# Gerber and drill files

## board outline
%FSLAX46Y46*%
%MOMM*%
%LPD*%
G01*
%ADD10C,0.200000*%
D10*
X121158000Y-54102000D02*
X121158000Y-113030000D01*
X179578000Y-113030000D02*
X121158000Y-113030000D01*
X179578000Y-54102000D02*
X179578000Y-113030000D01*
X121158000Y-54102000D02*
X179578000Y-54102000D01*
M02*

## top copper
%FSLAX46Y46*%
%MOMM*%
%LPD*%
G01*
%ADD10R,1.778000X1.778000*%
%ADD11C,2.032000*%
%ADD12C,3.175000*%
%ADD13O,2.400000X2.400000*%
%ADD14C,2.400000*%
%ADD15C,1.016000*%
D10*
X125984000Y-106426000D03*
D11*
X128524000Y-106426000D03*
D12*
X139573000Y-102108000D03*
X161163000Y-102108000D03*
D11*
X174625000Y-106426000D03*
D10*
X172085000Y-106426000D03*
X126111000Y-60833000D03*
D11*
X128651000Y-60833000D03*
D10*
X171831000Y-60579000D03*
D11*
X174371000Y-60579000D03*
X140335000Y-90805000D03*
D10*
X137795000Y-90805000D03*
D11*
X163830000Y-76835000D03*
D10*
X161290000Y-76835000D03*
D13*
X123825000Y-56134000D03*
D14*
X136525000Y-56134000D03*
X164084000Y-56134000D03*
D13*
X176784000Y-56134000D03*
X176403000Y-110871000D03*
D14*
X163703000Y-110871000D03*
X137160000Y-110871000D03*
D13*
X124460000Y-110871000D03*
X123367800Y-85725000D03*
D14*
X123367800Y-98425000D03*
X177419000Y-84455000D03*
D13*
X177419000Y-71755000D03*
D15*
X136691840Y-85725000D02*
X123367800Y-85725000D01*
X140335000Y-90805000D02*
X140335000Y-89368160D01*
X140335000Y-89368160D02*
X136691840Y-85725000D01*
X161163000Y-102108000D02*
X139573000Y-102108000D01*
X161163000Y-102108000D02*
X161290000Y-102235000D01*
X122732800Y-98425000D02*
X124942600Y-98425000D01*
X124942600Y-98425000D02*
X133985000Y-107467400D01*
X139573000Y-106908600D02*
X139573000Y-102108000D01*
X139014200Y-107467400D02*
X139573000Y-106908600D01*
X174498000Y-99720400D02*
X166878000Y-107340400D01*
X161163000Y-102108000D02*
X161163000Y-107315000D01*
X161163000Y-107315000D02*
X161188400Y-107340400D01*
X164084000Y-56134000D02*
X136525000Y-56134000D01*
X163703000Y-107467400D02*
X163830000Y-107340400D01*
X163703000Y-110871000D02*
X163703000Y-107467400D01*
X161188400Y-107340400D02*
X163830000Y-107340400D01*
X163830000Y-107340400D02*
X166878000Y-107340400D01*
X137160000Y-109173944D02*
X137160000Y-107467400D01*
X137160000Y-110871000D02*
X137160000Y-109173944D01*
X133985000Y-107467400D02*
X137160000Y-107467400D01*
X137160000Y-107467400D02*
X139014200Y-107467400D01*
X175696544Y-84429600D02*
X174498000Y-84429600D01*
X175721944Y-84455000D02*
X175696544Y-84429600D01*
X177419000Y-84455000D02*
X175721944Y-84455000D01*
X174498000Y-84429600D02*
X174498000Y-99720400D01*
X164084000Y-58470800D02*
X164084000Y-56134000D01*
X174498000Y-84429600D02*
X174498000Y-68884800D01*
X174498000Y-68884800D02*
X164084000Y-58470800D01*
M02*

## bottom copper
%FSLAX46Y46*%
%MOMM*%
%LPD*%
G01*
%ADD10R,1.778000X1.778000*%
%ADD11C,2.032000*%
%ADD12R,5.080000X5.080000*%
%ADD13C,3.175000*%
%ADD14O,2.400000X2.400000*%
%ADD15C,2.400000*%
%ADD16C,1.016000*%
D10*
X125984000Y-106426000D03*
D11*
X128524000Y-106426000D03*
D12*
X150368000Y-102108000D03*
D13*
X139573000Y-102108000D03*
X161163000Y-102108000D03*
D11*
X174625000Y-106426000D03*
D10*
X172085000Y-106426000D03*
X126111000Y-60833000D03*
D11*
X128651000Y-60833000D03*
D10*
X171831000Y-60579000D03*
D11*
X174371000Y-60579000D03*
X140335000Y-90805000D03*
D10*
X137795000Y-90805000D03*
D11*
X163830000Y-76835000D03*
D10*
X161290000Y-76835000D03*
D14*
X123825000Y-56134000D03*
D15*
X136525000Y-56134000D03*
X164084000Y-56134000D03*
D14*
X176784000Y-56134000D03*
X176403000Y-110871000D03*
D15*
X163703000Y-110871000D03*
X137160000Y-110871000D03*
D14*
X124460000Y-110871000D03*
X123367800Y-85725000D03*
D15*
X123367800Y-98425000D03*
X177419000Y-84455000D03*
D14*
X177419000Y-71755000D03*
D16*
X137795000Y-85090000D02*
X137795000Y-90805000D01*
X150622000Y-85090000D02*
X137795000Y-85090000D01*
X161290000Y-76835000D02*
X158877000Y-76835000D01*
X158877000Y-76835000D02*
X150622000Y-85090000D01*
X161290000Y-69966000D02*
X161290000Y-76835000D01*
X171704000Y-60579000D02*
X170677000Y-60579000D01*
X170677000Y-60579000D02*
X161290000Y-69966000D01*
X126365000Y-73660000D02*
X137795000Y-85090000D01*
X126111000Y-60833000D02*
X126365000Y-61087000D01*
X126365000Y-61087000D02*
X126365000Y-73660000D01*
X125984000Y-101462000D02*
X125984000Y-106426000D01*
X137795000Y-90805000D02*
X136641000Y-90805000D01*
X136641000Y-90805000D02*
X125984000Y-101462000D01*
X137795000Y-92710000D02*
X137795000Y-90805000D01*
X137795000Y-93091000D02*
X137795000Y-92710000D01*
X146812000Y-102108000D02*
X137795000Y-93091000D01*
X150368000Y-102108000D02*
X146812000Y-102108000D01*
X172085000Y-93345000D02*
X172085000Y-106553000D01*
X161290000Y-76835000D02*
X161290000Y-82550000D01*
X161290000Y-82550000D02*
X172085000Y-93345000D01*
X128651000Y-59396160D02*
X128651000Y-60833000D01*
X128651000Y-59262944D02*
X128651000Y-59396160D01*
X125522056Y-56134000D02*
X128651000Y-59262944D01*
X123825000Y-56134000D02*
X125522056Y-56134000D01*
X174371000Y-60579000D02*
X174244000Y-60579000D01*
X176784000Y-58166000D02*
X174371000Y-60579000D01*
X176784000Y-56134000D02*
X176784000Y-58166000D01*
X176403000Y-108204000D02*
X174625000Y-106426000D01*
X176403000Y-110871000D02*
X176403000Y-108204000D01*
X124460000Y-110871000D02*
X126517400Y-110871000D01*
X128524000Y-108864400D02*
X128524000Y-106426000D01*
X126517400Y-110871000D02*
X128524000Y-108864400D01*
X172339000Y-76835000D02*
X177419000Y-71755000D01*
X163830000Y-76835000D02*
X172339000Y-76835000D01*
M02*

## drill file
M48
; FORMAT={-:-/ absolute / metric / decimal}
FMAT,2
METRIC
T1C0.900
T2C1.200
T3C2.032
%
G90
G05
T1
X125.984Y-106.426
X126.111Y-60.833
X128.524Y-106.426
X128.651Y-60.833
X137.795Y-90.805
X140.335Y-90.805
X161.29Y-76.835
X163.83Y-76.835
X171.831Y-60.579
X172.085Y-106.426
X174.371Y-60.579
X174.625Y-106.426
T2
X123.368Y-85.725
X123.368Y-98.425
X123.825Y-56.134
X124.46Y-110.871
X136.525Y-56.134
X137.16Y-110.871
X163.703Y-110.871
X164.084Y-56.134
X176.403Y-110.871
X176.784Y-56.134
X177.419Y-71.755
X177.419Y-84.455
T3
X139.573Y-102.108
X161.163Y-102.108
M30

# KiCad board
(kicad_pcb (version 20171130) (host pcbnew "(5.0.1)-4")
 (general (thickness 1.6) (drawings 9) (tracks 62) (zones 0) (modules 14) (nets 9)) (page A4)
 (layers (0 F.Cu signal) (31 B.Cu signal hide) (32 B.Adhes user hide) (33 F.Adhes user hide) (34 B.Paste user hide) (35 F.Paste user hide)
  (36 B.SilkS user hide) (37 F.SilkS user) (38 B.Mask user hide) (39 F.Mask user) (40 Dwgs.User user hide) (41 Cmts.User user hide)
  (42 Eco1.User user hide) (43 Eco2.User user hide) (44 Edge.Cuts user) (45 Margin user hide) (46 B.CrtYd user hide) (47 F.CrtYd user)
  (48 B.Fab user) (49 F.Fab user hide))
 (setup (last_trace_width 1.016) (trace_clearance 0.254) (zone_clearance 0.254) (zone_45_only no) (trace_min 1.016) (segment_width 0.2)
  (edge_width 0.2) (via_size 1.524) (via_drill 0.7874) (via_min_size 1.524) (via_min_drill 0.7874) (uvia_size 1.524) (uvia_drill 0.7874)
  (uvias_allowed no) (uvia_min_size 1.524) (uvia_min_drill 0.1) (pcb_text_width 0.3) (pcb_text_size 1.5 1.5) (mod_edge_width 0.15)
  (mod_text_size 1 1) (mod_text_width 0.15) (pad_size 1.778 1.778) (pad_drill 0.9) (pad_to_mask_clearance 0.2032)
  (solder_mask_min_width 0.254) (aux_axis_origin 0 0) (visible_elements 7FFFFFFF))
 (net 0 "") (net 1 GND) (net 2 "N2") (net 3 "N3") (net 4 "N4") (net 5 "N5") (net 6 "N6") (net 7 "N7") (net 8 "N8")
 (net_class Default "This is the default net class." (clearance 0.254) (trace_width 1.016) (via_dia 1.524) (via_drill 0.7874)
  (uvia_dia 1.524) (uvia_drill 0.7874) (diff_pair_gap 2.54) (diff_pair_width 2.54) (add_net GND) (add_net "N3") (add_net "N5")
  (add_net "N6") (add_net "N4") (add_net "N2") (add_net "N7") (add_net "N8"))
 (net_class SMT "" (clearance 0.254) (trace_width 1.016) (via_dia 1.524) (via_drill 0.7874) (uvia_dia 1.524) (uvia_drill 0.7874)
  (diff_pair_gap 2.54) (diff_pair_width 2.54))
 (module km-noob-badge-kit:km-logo (layer F.Cu) (at 150.368 83.566)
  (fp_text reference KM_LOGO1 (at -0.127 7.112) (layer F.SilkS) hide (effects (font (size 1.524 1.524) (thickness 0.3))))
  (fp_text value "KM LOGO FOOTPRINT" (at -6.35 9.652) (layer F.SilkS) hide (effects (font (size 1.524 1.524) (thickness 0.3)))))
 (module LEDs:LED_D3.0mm (layer F.Cu) (at 125.984 106.426)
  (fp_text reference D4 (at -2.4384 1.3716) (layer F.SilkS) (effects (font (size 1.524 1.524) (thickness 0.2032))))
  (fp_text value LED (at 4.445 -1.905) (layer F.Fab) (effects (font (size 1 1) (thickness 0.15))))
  (pad 1 thru_hole rect (at 0 0) (size 1.778 1.778) (drill 0.9) (layers *.Cu *.Mask) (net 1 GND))
  (pad 2 thru_hole circle (at 2.54 0) (size 2.032 2.032) (drill 0.9) (layers *.Cu *.Mask) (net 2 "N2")))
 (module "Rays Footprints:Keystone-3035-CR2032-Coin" (layer B.Cu) (at 150.368 102.108 180)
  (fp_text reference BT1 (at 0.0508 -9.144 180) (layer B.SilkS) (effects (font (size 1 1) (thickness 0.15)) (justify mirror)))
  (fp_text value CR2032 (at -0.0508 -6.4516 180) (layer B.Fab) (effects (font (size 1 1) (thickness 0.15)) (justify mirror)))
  (pad 2 smd rect (at 0 0 180) (size 5.08 5.08) (layers B.Cu B.Paste B.Mask) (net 1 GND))
  (pad 1 thru_hole circle (at 10.795 0 180) (size 3.175 3.175) (drill 2.032) (layers *.Cu *.Mask) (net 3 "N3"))
  (pad 1 thru_hole circle (at -10.795 0 90) (size 3.175 3.175) (drill 2.032) (layers *.Cu *.Mask) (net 3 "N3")))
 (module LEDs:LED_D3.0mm (layer F.Cu) (at 172.085 106.426)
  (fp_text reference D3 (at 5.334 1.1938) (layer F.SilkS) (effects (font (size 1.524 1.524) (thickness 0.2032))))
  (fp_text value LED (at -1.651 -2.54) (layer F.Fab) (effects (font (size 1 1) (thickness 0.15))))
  (pad 2 thru_hole circle (at 2.54 0) (size 2.032 2.032) (drill 0.9) (layers *.Cu *.Mask) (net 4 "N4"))
  (pad 1 thru_hole rect (at 0 0) (size 1.778 1.778) (drill 0.9) (layers *.Cu *.Mask) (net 1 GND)))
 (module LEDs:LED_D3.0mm (layer F.Cu) (at 126.111 60.833)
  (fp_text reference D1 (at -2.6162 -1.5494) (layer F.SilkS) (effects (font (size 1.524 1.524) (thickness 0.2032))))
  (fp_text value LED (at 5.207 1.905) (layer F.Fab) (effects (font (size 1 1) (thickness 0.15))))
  (pad 1 thru_hole rect (at 0 0) (size 1.778 1.778) (drill 0.9) (layers *.Cu *.Mask) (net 1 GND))
  (pad 2 thru_hole circle (at 2.54 0) (size 2.032 2.032) (drill 0.9) (layers *.Cu *.Mask) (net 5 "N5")))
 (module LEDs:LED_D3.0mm (layer F.Cu) (at 171.831 60.579)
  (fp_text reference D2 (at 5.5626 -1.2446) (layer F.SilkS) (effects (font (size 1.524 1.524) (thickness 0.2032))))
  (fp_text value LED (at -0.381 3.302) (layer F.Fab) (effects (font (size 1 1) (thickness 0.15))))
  (pad 1 thru_hole rect (at 0 0) (size 1.778 1.778) (drill 0.9) (layers *.Cu *.Mask) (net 1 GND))
  (pad 2 thru_hole circle (at 2.54 0) (size 2.032 2.032) (drill 0.9) (layers *.Cu *.Mask) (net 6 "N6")))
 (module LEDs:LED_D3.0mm (layer F.Cu) (at 137.795 90.805)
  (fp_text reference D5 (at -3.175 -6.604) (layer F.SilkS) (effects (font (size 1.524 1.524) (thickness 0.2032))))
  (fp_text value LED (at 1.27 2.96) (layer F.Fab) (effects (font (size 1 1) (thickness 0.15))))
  (pad 2 thru_hole circle (at 2.54 0) (size 2.032 2.032) (drill 0.9) (layers *.Cu *.Mask) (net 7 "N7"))
  (pad 1 thru_hole rect (at 0 0) (size 1.778 1.778) (drill 0.9) (layers *.Cu *.Mask) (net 1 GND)))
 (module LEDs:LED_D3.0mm (layer F.Cu) (at 161.29 76.835)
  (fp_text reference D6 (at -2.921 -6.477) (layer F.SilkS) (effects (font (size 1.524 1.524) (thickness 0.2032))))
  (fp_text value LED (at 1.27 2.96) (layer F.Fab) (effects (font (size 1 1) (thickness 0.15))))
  (pad 2 thru_hole circle (at 2.54 0) (size 2.032 2.032) (drill 0.9) (layers *.Cu *.Mask) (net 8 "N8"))
  (pad 1 thru_hole rect (at 0 0) (size 1.778 1.778) (drill 0.9) (layers *.Cu *.Mask) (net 1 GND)))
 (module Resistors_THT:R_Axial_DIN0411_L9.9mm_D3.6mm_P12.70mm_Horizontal (layer F.Cu) (at 136.525 56.134 180)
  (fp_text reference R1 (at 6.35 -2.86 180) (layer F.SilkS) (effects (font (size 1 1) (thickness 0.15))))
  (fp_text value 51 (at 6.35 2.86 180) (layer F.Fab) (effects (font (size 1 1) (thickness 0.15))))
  (pad 2 thru_hole oval (at 12.7 0 180) (size 2.4 2.4) (drill 1.2) (layers *.Cu *.Mask) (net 5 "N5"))
  (pad 1 thru_hole circle (at 0 0 180) (size 2.4 2.4) (drill 1.2) (layers *.Cu *.Mask) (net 3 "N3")))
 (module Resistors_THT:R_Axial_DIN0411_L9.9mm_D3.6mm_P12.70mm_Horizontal (layer F.Cu) (at 164.084 56.134)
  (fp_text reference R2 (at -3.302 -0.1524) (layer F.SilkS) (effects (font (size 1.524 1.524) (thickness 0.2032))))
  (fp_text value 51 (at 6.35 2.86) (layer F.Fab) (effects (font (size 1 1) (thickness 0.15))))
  (pad 1 thru_hole circle (at 0 0) (size 2.4 2.4) (drill 1.2) (layers *.Cu *.Mask) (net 3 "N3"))
  (pad 2 thru_hole oval (at 12.7 0) (size 2.4 2.4) (drill 1.2) (layers *.Cu *.Mask) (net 6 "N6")))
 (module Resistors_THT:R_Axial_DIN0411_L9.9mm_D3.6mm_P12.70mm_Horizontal (layer F.Cu) (at 163.703 110.871)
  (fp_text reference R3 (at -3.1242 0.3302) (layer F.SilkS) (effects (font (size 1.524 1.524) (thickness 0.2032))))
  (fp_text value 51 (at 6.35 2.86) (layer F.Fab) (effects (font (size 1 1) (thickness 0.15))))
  (pad 2 thru_hole oval (at 12.7 0) (size 2.4 2.4) (drill 1.2) (layers *.Cu *.Mask) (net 4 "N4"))
  (pad 1 thru_hole circle (at 0 0) (size 2.4 2.4) (drill 1.2) (layers *.Cu *.Mask) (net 3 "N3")))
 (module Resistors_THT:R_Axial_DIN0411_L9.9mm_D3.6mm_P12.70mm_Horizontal (layer F.Cu) (at 137.16 110.871 180)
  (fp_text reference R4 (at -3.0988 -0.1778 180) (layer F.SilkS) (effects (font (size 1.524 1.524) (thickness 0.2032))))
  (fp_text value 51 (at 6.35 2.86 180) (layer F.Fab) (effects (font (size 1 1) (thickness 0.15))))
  (pad 1 thru_hole circle (at 0 0 180) (size 2.4 2.4) (drill 1.2) (layers *.Cu *.Mask) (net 3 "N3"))
  (pad 2 thru_hole oval (at 12.7 0 180) (size 2.4 2.4) (drill 1.2) (layers *.Cu *.Mask) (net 2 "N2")))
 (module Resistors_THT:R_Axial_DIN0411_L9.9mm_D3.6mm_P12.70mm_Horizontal (layer F.Cu) (at 123.3678 98.425 90)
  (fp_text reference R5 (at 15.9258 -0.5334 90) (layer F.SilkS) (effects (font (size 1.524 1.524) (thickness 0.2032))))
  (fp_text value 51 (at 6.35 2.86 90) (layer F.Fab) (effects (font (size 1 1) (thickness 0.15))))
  (pad 2 thru_hole oval (at 12.7 0 90) (size 2.4 2.4) (drill 1.2) (layers *.Cu *.Mask) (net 7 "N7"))
  (pad 1 thru_hole circle (at 0 0 90) (size 2.4 2.4) (drill 1.2) (layers *.Cu *.Mask) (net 3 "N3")))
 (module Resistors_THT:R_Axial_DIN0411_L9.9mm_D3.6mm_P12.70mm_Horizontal (layer F.Cu) (at 177.419 84.455 90)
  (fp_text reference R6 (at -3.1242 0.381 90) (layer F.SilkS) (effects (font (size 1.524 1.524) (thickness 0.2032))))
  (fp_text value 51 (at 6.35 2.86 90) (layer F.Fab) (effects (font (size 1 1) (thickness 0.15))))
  (pad 1 thru_hole circle (at 0 0 90) (size 2.4 2.4) (drill 1.2) (layers *.Cu *.Mask) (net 3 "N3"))
  (pad 2 thru_hole oval (at 12.7 0 90) (size 2.4 2.4) (drill 1.2) (layers *.Cu *.Mask) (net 8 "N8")))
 (gr_line (start 121.158 54.102) (end 121.158 113.03) (layer Edge.Cuts) (width 0.2))
 (gr_line (start 179.578 113.03) (end 121.158 113.03) (layer Edge.Cuts) (width 0.2))
 (gr_line (start 179.578 54.102) (end 179.578 113.03) (layer Edge.Cuts) (width 0.2))
 (gr_line (start 121.158 54.102) (end 179.578 54.102) (layer Edge.Cuts) (width 0.2))
 (segment (start 137.795 85.09) (end 137.795 90.805) (width 1.016) (layer B.Cu) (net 1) (status 20))
 (segment (start 150.622 85.09) (end 137.795 85.09) (width 1.016) (layer B.Cu) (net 1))
 (segment (start 161.29 76.835) (end 158.877 76.835) (width 1.016) (layer B.Cu) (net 1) (status 10))
 (segment (start 158.877 76.835) (end 150.622 85.09) (width 1.016) (layer B.Cu) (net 1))
 (segment (start 161.29 69.966) (end 161.29 76.835) (width 1.016) (layer B.Cu) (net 1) (status 20))
 (segment (start 171.704 60.579) (end 170.677 60.579) (width 1.016) (layer B.Cu) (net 1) (status 10))
 (segment (start 170.677 60.579) (end 161.29 69.966) (width 1.016) (layer B.Cu) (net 1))
 (segment (start 126.365 73.66) (end 137.795 85.09) (width 1.016) (layer B.Cu) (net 1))
 (segment (start 126.111 60.833) (end 126.365 61.087) (width 1.016) (layer B.Cu) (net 1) (status 30))
 (segment (start 126.365 61.087) (end 126.365 73.66) (width 1.016) (layer B.Cu) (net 1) (status 10))
 (segment (start 125.984 101.462) (end 125.984 106.426) (width 1.016) (layer B.Cu) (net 1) (status 20))
 (segment (start 137.795 90.805) (end 136.641 90.805) (width 1.016) (layer B.Cu) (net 1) (status 10))
 (segment (start 136.641 90.805) (end 125.984 101.462) (width 1.016) (layer B.Cu) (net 1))
 (segment (start 137.795 92.71) (end 137.795 90.805) (width 1.016) (layer B.Cu) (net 1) (status 20))
 (segment (start 137.795 93.091) (end 137.795 92.71) (width 1.016) (layer B.Cu) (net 1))
 (segment (start 146.812 102.108) (end 137.795 93.091) (width 1.016) (layer B.Cu) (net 1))
 (segment (start 150.368 102.108) (end 146.812 102.108) (width 1.016) (layer B.Cu) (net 1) (status 10))
 (segment (start 172.085 93.345) (end 172.085 106.553) (width 1.016) (layer B.Cu) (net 1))
 (segment (start 161.29 76.835) (end 161.29 82.55) (width 1.016) (layer B.Cu) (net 1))
 (segment (start 161.29 82.55) (end 172.085 93.345) (width 1.016) (layer B.Cu) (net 1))
 (segment (start 128.651 59.39616) (end 128.651 60.833) (width 1.016) (layer B.Cu) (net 5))
 (segment (start 128.651 59.262944) (end 128.651 59.39616) (width 1.016) (layer B.Cu) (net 5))
 (segment (start 125.522056 56.134) (end 128.651 59.262944) (width 1.016) (layer B.Cu) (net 5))
 (segment (start 123.825 56.134) (end 125.522056 56.134) (width 1.016) (layer B.Cu) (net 5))
 (segment (start 174.371 60.579) (end 174.244 60.579) (width 1.016) (layer B.Cu) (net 6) (status 30))
 (segment (start 176.784 58.166) (end 174.371 60.579) (width 1.016) (layer B.Cu) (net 6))
 (segment (start 176.784 56.134) (end 176.784 58.166) (width 1.016) (layer B.Cu) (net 6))
 (segment (start 176.403 108.204) (end 174.625 106.426) (width 1.016) (layer B.Cu) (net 4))
 (segment (start 176.403 110.871) (end 176.403 108.204) (width 1.016) (layer B.Cu) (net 4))
 (segment (start 124.46 110.871) (end 126.5174 110.871) (width 1.016) (layer B.Cu) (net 2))
 (segment (start 128.524 108.8644) (end 128.524 106.426) (width 1.016) (layer B.Cu) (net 2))
 (segment (start 126.5174 110.871) (end 128.524 108.8644) (width 1.016) (layer B.Cu) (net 2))
 (segment (start 136.69184 85.725) (end 123.3678 85.725) (width 1.016) (layer F.Cu) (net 7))
 (segment (start 140.335 90.805) (end 140.335 89.36816) (width 1.016) (layer F.Cu) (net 7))
 (segment (start 140.335 89.36816) (end 136.69184 85.725) (width 1.016) (layer F.Cu) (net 7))
 (segment (start 172.339 76.835) (end 177.419 71.755) (width 1.016) (layer B.Cu) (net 8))
 (segment (start 163.83 76.835) (end 172.339 76.835) (width 1.016) (layer B.Cu) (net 8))
 (segment (start 161.163 102.108) (end 139.573 102.108) (width 1.016) (layer F.Cu) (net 3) (status 30))
 (segment (start 161.163 102.108) (end 161.29 102.235) (width 1.016) (layer F.Cu) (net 3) (status 30))
 (segment (start 122.7328 98.425) (end 124.9426 98.425) (width 1.016) (layer F.Cu) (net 3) (status 10))
 (segment (start 124.9426 98.425) (end 133.985 107.4674) (width 1.016) (layer F.Cu) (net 3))
 (segment (start 139.573 106.9086) (end 139.573 102.108) (width 1.016) (layer F.Cu) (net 3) (status 20))
 (segment (start 139.0142 107.4674) (end 139.573 106.9086) (width 1.016) (layer F.Cu) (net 3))
 (segment (start 174.498 99.7204) (end 166.878 107.3404) (width 1.016) (layer F.Cu) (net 3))
 (segment (start 161.163 102.108) (end 161.163 107.315) (width 1.016) (layer F.Cu) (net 3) (status 10))
 (segment (start 161.163 107.315) (end 161.1884 107.3404) (width 1.016) (layer F.Cu) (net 3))
 (segment (start 164.084 56.134) (end 136.525 56.134) (width 1.016) (layer F.Cu) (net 3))
 (segment (start 163.703 107.4674) (end 163.83 107.3404) (width 1.016) (layer F.Cu) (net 3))
 (segment (start 163.703 110.871) (end 163.703 107.4674) (width 1.016) (layer F.Cu) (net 3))
 (segment (start 161.1884 107.3404) (end 163.83 107.3404) (width 1.016) (layer F.Cu) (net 3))
 (segment (start 163.83 107.3404) (end 166.878 107.3404) (width 1.016) (layer F.Cu) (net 3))
 (segment (start 137.16 109.173944) (end 137.16 107.4674) (width 1.016) (layer F.Cu) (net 3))
 (segment (start 137.16 110.871) (end 137.16 109.173944) (width 1.016) (layer F.Cu) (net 3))
 (segment (start 133.985 107.4674) (end 137.16 107.4674) (width 1.016) (layer F.Cu) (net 3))
 (segment (start 137.16 107.4674) (end 139.0142 107.4674) (width 1.016) (layer F.Cu) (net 3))
 (segment (start 175.696544 84.4296) (end 174.498 84.4296) (width 1.016) (layer F.Cu) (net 3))
 (segment (start 175.721944 84.455) (end 175.696544 84.4296) (width 1.016) (layer F.Cu) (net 3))
 (segment (start 177.419 84.455) (end 175.721944 84.455) (width 1.016) (layer F.Cu) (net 3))
 (segment (start 174.498 84.4296) (end 174.498 99.7204) (width 1.016) (layer F.Cu) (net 3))
 (segment (start 164.084 58.4708) (end 164.084 56.134) (width 1.016) (layer F.Cu) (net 3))
 (segment (start 174.498 84.4296) (end 174.498 68.8848) (width 1.016) (layer F.Cu) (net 3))
 (segment (start 174.498 68.8848) (end 164.084 58.4708) (width 1.016) (layer F.Cu) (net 3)))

